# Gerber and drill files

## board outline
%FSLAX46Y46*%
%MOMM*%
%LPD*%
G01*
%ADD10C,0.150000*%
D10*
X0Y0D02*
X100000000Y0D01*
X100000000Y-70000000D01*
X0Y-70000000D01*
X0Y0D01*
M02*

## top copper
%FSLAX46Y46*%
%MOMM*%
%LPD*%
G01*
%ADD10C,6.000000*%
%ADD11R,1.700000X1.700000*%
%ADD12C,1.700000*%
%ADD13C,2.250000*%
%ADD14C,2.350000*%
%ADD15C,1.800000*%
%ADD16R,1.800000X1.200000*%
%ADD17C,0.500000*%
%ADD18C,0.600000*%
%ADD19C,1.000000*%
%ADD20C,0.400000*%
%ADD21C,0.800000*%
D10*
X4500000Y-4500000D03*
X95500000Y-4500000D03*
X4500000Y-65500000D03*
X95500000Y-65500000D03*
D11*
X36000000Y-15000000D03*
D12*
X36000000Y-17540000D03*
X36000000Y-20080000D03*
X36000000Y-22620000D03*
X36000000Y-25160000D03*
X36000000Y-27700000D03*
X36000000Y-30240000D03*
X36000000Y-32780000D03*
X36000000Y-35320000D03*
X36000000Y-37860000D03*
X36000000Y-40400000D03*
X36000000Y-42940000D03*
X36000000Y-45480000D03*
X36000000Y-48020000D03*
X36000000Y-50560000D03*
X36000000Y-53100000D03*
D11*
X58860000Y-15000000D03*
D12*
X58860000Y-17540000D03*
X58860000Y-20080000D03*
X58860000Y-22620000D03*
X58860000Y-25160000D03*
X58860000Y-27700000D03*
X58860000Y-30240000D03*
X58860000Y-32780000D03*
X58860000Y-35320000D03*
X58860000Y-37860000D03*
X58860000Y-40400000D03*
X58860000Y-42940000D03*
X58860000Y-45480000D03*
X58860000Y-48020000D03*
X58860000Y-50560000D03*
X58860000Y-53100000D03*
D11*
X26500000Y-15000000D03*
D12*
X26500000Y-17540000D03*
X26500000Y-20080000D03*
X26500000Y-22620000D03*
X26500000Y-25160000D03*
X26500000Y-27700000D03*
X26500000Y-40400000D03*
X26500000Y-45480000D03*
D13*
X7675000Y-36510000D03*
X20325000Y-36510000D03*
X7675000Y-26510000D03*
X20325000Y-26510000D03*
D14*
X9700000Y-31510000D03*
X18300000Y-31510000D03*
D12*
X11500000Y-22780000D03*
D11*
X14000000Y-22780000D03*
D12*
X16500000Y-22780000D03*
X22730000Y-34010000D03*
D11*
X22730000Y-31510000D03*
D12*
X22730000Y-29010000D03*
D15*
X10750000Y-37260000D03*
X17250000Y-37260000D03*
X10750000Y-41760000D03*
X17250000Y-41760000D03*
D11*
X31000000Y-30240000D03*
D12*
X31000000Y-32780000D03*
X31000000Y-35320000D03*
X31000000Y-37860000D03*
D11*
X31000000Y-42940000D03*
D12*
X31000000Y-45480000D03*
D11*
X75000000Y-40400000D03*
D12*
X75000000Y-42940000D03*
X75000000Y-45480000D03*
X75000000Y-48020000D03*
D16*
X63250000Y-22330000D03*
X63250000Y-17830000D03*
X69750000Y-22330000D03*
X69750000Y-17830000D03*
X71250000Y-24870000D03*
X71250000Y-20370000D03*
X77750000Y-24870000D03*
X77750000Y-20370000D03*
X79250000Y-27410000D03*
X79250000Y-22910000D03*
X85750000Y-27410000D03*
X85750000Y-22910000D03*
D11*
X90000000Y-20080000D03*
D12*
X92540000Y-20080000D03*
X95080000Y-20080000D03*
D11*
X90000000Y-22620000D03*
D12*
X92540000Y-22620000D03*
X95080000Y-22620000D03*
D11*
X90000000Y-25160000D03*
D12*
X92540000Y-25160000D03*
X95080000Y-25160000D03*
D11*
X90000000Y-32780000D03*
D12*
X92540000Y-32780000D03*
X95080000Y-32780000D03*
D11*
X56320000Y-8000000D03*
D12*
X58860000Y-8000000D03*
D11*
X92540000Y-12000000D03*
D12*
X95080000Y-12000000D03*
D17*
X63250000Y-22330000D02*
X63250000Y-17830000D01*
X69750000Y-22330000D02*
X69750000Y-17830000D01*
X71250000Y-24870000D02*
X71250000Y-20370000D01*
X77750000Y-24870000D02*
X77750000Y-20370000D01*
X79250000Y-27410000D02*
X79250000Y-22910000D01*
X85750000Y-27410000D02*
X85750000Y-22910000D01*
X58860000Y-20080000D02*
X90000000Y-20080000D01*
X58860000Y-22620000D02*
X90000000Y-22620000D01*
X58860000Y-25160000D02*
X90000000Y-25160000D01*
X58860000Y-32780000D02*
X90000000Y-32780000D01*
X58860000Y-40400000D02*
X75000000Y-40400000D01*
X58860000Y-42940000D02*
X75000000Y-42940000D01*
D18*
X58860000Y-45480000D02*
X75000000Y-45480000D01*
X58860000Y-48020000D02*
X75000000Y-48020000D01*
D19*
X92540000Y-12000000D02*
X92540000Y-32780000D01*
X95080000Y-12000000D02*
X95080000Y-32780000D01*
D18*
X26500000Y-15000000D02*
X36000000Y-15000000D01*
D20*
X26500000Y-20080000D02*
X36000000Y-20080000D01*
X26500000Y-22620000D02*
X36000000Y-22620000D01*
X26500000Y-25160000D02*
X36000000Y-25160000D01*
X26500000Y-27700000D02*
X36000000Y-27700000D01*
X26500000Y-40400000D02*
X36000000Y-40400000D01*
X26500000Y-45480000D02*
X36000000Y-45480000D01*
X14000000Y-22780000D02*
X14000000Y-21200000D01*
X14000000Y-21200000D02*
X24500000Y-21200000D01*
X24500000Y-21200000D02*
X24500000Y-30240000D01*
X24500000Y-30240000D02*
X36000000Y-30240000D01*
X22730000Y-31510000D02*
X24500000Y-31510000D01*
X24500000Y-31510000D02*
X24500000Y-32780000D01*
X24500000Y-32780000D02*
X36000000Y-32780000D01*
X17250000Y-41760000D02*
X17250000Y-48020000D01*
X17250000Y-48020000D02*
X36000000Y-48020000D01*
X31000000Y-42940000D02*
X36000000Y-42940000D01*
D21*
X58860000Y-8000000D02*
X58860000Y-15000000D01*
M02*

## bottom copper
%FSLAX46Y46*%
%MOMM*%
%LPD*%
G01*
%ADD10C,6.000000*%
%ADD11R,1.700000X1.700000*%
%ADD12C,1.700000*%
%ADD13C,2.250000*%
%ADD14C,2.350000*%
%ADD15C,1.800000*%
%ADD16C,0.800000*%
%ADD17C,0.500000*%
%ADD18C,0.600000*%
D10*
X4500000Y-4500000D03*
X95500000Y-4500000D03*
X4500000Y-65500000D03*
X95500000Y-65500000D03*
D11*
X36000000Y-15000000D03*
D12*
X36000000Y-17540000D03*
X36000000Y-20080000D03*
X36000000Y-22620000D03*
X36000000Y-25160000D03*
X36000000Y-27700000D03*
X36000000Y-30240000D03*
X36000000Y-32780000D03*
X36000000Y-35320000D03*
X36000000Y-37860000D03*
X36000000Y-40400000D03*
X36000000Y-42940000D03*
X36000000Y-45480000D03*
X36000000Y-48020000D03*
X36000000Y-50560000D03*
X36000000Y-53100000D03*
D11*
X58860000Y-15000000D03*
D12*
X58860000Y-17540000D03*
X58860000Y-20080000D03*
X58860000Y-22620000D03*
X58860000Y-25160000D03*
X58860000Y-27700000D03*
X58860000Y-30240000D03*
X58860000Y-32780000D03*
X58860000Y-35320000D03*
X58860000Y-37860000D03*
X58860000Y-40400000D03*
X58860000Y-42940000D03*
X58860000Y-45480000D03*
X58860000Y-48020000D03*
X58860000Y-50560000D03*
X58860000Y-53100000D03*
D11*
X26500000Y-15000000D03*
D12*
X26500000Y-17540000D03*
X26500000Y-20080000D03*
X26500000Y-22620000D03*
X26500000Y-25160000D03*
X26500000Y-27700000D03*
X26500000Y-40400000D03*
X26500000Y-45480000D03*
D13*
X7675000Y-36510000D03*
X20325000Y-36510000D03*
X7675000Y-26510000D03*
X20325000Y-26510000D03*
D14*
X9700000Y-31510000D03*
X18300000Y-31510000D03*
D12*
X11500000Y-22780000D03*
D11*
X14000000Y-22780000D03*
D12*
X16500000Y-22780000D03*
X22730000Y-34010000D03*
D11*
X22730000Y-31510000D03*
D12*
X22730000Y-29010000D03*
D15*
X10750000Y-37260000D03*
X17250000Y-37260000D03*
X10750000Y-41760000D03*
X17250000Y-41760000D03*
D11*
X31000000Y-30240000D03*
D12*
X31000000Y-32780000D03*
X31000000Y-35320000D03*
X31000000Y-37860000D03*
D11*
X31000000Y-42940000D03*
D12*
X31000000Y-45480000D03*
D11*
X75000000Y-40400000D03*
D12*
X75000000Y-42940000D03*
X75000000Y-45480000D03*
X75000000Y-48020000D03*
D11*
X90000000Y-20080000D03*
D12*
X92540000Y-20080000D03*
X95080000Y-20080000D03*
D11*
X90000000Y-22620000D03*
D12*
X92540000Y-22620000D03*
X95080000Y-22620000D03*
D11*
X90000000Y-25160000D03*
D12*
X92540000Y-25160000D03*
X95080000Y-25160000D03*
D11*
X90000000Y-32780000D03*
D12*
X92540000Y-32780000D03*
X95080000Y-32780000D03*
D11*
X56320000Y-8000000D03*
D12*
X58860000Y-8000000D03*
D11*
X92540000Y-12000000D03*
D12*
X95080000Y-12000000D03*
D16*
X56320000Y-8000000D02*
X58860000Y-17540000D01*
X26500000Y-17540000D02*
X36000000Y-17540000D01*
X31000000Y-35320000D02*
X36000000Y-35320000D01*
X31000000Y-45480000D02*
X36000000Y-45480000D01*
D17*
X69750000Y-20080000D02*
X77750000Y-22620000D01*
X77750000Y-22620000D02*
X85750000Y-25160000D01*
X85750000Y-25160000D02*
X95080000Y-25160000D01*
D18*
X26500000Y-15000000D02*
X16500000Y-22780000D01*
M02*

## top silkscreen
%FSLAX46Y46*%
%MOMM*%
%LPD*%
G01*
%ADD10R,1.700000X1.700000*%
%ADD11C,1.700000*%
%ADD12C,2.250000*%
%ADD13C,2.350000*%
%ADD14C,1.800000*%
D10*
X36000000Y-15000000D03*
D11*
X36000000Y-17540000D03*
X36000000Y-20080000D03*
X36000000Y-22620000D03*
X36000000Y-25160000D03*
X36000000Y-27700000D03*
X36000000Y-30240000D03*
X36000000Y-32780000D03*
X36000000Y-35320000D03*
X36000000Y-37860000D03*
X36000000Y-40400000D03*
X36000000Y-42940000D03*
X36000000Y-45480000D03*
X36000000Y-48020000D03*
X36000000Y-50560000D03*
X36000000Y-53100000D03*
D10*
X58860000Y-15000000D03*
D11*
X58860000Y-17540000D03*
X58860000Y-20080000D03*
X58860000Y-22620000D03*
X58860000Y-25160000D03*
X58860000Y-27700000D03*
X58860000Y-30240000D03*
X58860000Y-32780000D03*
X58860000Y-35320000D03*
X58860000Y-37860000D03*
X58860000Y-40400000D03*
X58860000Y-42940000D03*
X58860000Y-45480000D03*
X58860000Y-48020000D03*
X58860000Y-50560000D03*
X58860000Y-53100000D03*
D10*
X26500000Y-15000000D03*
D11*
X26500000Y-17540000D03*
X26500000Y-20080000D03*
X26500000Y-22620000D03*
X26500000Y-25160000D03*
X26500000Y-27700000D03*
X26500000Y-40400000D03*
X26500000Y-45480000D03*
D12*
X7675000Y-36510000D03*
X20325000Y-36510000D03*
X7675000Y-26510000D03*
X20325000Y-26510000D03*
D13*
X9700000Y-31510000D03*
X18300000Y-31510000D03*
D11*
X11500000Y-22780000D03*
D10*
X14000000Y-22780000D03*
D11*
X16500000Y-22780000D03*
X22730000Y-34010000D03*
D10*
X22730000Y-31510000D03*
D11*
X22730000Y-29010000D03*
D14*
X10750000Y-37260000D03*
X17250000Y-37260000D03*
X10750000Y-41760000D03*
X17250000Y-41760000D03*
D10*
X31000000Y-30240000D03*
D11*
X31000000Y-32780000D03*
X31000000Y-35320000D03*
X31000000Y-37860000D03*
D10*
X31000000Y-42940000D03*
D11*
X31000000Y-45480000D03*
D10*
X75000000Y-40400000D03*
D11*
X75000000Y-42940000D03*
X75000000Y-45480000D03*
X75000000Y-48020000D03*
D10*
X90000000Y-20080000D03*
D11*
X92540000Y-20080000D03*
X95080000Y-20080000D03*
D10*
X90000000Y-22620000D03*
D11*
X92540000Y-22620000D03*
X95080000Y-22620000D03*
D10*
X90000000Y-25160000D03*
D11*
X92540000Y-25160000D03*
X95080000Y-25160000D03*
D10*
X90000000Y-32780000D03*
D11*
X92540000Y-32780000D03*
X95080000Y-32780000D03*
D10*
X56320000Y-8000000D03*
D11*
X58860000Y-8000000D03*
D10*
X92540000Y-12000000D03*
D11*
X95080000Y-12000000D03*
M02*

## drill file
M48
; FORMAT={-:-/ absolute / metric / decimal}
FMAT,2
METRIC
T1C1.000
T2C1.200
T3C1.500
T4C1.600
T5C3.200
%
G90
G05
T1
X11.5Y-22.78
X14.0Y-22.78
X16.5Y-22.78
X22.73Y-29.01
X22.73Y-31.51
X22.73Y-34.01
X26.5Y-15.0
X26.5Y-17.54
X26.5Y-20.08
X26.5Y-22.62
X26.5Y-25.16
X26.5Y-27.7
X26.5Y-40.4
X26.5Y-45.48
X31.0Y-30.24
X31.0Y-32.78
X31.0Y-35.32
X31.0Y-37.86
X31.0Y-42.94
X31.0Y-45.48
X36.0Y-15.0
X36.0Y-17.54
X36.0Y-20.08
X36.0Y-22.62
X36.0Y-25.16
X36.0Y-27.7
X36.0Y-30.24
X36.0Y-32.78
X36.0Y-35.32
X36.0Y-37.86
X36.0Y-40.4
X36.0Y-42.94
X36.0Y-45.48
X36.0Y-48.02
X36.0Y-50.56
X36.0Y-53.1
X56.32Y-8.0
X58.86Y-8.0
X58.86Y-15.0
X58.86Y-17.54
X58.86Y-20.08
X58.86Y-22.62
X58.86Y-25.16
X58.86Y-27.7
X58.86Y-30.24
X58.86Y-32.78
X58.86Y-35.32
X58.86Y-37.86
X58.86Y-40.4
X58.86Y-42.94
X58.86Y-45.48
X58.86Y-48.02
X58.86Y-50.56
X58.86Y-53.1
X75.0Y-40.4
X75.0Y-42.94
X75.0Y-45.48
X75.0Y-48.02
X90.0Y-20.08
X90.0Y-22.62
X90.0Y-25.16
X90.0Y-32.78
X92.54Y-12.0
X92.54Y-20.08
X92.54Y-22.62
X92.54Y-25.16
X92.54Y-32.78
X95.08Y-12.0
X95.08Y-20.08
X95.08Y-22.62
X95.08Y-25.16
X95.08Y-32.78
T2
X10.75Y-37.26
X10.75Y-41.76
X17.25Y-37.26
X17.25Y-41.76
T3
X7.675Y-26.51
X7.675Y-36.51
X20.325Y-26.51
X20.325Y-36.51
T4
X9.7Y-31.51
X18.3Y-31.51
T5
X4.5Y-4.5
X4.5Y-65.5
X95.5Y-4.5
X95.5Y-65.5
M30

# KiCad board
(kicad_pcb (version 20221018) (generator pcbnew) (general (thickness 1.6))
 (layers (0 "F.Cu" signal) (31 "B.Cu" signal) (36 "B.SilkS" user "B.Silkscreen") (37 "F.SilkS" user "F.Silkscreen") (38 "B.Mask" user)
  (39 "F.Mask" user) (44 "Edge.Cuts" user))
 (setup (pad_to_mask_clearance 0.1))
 (gr_rect (start 0 0) (end 100.0 70.0) (layer "Edge.Cuts") (width 0.15) (fill none))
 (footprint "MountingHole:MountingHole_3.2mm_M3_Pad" (layer "F.Cu") (at 4.5 4.5)
  (pad "" np_thru_hole circle (at 0 0) (size 6.0 6.0) (drill 3.2) (layers *.Cu *.Mask)))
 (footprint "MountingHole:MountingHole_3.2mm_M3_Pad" (layer "F.Cu") (at 95.5 4.5)
  (pad "" np_thru_hole circle (at 0 0) (size 6.0 6.0) (drill 3.2) (layers *.Cu *.Mask)))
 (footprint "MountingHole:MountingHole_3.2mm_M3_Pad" (layer "F.Cu") (at 4.5 65.5)
  (pad "" np_thru_hole circle (at 0 0) (size 6.0 6.0) (drill 3.2) (layers *.Cu *.Mask)))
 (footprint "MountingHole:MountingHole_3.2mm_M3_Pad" (layer "F.Cu") (at 95.5 65.5)
  (pad "" np_thru_hole circle (at 0 0) (size 6.0 6.0) (drill 3.2) (layers *.Cu *.Mask)))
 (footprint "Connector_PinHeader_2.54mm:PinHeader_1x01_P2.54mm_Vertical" (layer "F.Cu") (at 36.0 15.0)
  (pad "1" thru_hole rect (at 0 0) (size 1.7 1.7) (drill 1.0) (layers *.Cu *.Mask "F.SilkS")))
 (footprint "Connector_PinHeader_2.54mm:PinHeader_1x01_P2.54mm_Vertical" (layer "F.Cu") (at 36.0 17.54)
  (pad "1" thru_hole circle (at 0 0) (size 1.7 1.7) (drill 1.0) (layers *.Cu *.Mask "F.SilkS")))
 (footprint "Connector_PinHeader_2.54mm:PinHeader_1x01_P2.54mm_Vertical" (layer "F.Cu") (at 36.0 20.08)
  (pad "1" thru_hole circle (at 0 0) (size 1.7 1.7) (drill 1.0) (layers *.Cu *.Mask "F.SilkS")))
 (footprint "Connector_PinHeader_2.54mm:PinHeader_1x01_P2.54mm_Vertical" (layer "F.Cu") (at 36.0 22.62)
  (pad "1" thru_hole circle (at 0 0) (size 1.7 1.7) (drill 1.0) (layers *.Cu *.Mask "F.SilkS")))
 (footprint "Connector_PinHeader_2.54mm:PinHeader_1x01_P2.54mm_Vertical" (layer "F.Cu") (at 36.0 25.16)
  (pad "1" thru_hole circle (at 0 0) (size 1.7 1.7) (drill 1.0) (layers *.Cu *.Mask "F.SilkS")))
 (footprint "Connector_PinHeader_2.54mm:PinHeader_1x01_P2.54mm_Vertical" (layer "F.Cu") (at 36.0 27.7)
  (pad "1" thru_hole circle (at 0 0) (size 1.7 1.7) (drill 1.0) (layers *.Cu *.Mask "F.SilkS")))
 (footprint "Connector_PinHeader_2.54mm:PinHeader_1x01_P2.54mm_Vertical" (layer "F.Cu") (at 36.0 30.240000000000002)
  (pad "1" thru_hole circle (at 0 0) (size 1.7 1.7) (drill 1.0) (layers *.Cu *.Mask "F.SilkS")))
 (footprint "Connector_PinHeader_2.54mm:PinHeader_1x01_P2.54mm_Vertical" (layer "F.Cu") (at 36.0 32.78)
  (pad "1" thru_hole circle (at 0 0) (size 1.7 1.7) (drill 1.0) (layers *.Cu *.Mask "F.SilkS")))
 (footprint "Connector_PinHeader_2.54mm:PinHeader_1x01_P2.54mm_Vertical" (layer "F.Cu") (at 36.0 35.32)
  (pad "1" thru_hole circle (at 0 0) (size 1.7 1.7) (drill 1.0) (layers *.Cu *.Mask "F.SilkS")))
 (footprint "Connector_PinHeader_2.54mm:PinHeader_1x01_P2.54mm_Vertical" (layer "F.Cu") (at 36.0 37.86)
  (pad "1" thru_hole circle (at 0 0) (size 1.7 1.7) (drill 1.0) (layers *.Cu *.Mask "F.SilkS")))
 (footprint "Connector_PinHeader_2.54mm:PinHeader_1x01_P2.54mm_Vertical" (layer "F.Cu") (at 36.0 40.4)
  (pad "1" thru_hole circle (at 0 0) (size 1.7 1.7) (drill 1.0) (layers *.Cu *.Mask "F.SilkS")))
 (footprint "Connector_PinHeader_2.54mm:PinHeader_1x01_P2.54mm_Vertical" (layer "F.Cu") (at 36.0 42.94)
  (pad "1" thru_hole circle (at 0 0) (size 1.7 1.7) (drill 1.0) (layers *.Cu *.Mask "F.SilkS")))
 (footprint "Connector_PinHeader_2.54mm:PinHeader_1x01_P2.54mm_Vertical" (layer "F.Cu") (at 36.0 45.480000000000004)
  (pad "1" thru_hole circle (at 0 0) (size 1.7 1.7) (drill 1.0) (layers *.Cu *.Mask "F.SilkS")))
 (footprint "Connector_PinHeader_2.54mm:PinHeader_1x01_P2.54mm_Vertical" (layer "F.Cu") (at 36.0 48.02)
  (pad "1" thru_hole circle (at 0 0) (size 1.7 1.7) (drill 1.0) (layers *.Cu *.Mask "F.SilkS")))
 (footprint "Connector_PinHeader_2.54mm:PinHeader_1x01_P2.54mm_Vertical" (layer "F.Cu") (at 36.0 50.56)
  (pad "1" thru_hole circle (at 0 0) (size 1.7 1.7) (drill 1.0) (layers *.Cu *.Mask "F.SilkS")))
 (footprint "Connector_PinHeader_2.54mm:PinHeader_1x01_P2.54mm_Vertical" (layer "F.Cu") (at 36.0 53.1)
  (pad "1" thru_hole circle (at 0 0) (size 1.7 1.7) (drill 1.0) (layers *.Cu *.Mask "F.SilkS")))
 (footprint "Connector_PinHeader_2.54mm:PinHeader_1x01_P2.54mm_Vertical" (layer "F.Cu") (at 58.86 15.0)
  (pad "1" thru_hole rect (at 0 0) (size 1.7 1.7) (drill 1.0) (layers *.Cu *.Mask "F.SilkS")))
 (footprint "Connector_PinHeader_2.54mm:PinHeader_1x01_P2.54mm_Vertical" (layer "F.Cu") (at 58.86 17.54)
  (pad "1" thru_hole circle (at 0 0) (size 1.7 1.7) (drill 1.0) (layers *.Cu *.Mask "F.SilkS")))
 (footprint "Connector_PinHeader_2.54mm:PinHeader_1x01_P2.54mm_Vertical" (layer "F.Cu") (at 58.86 20.08)
  (pad "1" thru_hole circle (at 0 0) (size 1.7 1.7) (drill 1.0) (layers *.Cu *.Mask "F.SilkS")))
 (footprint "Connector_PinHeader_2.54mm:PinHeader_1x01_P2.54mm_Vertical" (layer "F.Cu") (at 58.86 22.62)
  (pad "1" thru_hole circle (at 0 0) (size 1.7 1.7) (drill 1.0) (layers *.Cu *.Mask "F.SilkS")))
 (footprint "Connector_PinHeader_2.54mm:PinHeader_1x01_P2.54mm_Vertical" (layer "F.Cu") (at 58.86 25.16)
  (pad "1" thru_hole circle (at 0 0) (size 1.7 1.7) (drill 1.0) (layers *.Cu *.Mask "F.SilkS")))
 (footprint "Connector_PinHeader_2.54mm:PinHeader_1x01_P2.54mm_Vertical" (layer "F.Cu") (at 58.86 27.7)
  (pad "1" thru_hole circle (at 0 0) (size 1.7 1.7) (drill 1.0) (layers *.Cu *.Mask "F.SilkS")))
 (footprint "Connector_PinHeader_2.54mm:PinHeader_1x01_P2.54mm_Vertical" (layer "F.Cu") (at 58.86 30.240000000000002)
  (pad "1" thru_hole circle (at 0 0) (size 1.7 1.7) (drill 1.0) (layers *.Cu *.Mask "F.SilkS")))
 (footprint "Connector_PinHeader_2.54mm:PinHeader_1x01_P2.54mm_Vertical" (layer "F.Cu") (at 58.86 32.78)
  (pad "1" thru_hole circle (at 0 0) (size 1.7 1.7) (drill 1.0) (layers *.Cu *.Mask "F.SilkS")))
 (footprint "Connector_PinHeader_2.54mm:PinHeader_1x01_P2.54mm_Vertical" (layer "F.Cu") (at 58.86 35.32)
  (pad "1" thru_hole circle (at 0 0) (size 1.7 1.7) (drill 1.0) (layers *.Cu *.Mask "F.SilkS")))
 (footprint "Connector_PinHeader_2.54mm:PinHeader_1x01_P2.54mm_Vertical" (layer "F.Cu") (at 58.86 37.86)
  (pad "1" thru_hole circle (at 0 0) (size 1.7 1.7) (drill 1.0) (layers *.Cu *.Mask "F.SilkS")))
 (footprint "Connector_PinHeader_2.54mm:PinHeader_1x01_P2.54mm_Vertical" (layer "F.Cu") (at 58.86 40.4)
  (pad "1" thru_hole circle (at 0 0) (size 1.7 1.7) (drill 1.0) (layers *.Cu *.Mask "F.SilkS")))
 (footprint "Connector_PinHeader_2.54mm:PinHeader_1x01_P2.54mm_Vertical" (layer "F.Cu") (at 58.86 42.94)
  (pad "1" thru_hole circle (at 0 0) (size 1.7 1.7) (drill 1.0) (layers *.Cu *.Mask "F.SilkS")))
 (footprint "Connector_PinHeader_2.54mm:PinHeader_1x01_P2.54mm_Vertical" (layer "F.Cu") (at 58.86 45.480000000000004)
  (pad "1" thru_hole circle (at 0 0) (size 1.7 1.7) (drill 1.0) (layers *.Cu *.Mask "F.SilkS")))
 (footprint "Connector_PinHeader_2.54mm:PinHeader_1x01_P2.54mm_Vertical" (layer "F.Cu") (at 58.86 48.02)
  (pad "1" thru_hole circle (at 0 0) (size 1.7 1.7) (drill 1.0) (layers *.Cu *.Mask "F.SilkS")))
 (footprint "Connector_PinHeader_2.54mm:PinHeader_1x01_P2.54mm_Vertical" (layer "F.Cu") (at 58.86 50.56)
  (pad "1" thru_hole circle (at 0 0) (size 1.7 1.7) (drill 1.0) (layers *.Cu *.Mask "F.SilkS")))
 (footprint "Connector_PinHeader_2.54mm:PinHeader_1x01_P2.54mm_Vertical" (layer "F.Cu") (at 58.86 53.1)
  (pad "1" thru_hole circle (at 0 0) (size 1.7 1.7) (drill 1.0) (layers *.Cu *.Mask "F.SilkS")))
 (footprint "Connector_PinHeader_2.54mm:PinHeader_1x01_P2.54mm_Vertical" (layer "F.Cu") (at 26.5 15.0)
  (pad "1" thru_hole rect (at 0 0) (size 1.7 1.7) (drill 1.0) (layers *.Cu *.Mask "F.SilkS")))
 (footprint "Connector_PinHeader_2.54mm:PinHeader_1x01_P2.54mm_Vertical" (layer "F.Cu") (at 26.5 17.54)
  (pad "1" thru_hole circle (at 0 0) (size 1.7 1.7) (drill 1.0) (layers *.Cu *.Mask "F.SilkS")))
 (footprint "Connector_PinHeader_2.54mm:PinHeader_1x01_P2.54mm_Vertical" (layer "F.Cu") (at 26.5 20.08)
  (pad "1" thru_hole circle (at 0 0) (size 1.7 1.7) (drill 1.0) (layers *.Cu *.Mask "F.SilkS")))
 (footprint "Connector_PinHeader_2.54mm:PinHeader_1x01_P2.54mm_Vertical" (layer "F.Cu") (at 26.5 22.62)
  (pad "1" thru_hole circle (at 0 0) (size 1.7 1.7) (drill 1.0) (layers *.Cu *.Mask "F.SilkS")))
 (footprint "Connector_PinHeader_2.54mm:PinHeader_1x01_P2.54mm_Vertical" (layer "F.Cu") (at 26.5 25.16)
  (pad "1" thru_hole circle (at 0 0) (size 1.7 1.7) (drill 1.0) (layers *.Cu *.Mask "F.SilkS")))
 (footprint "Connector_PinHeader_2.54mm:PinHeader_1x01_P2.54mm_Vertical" (layer "F.Cu") (at 26.5 27.7)
  (pad "1" thru_hole circle (at 0 0) (size 1.7 1.7) (drill 1.0) (layers *.Cu *.Mask "F.SilkS")))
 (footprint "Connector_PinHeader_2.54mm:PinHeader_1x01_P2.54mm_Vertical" (layer "F.Cu") (at 26.5 40.4)
  (pad "1" thru_hole circle (at 0 0) (size 1.7 1.7) (drill 1.0) (layers *.Cu *.Mask "F.SilkS")))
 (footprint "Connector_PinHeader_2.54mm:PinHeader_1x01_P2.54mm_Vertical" (layer "F.Cu") (at 26.5 45.48)
  (pad "1" thru_hole circle (at 0 0) (size 1.7 1.7) (drill 1.0) (layers *.Cu *.Mask "F.SilkS")))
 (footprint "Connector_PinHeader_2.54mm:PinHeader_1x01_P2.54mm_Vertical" (layer "F.Cu") (at 7.675 36.510000000000005)
  (pad "1" thru_hole circle (at 0 0) (size 2.25 2.25) (drill 1.5) (layers *.Cu *.Mask "F.SilkS")))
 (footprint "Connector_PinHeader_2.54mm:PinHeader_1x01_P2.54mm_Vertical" (layer "F.Cu") (at 20.325 36.510000000000005)
  (pad "1" thru_hole circle (at 0 0) (size 2.25 2.25) (drill 1.5) (layers *.Cu *.Mask "F.SilkS")))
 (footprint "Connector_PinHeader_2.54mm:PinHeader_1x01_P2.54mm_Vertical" (layer "F.Cu") (at 7.675 26.51)
  (pad "1" thru_hole circle (at 0 0) (size 2.25 2.25) (drill 1.5) (layers *.Cu *.Mask "F.SilkS")))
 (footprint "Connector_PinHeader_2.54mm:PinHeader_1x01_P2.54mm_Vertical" (layer "F.Cu") (at 20.325 26.51)
  (pad "1" thru_hole circle (at 0 0) (size 2.25 2.25) (drill 1.5) (layers *.Cu *.Mask "F.SilkS")))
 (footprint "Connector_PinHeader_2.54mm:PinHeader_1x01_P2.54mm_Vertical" (layer "F.Cu") (at 9.7 31.51)
  (pad "1" thru_hole circle (at 0 0) (size 2.35 2.35) (drill 1.6) (layers *.Cu *.Mask "F.SilkS")))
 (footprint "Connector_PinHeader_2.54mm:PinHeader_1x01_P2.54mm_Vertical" (layer "F.Cu") (at 18.3 31.51)
  (pad "1" thru_hole circle (at 0 0) (size 2.35 2.35) (drill 1.6) (layers *.Cu *.Mask "F.SilkS")))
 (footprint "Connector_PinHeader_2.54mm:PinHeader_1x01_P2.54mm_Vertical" (layer "F.Cu") (at 11.5 22.78)
  (pad "1" thru_hole circle (at 0 0) (size 1.7 1.7) (drill 1.0) (layers *.Cu *.Mask "F.SilkS")))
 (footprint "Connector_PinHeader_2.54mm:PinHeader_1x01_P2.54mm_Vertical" (layer "F.Cu") (at 14.0 22.78)
  (pad "1" thru_hole rect (at 0 0) (size 1.7 1.7) (drill 1.0) (layers *.Cu *.Mask "F.SilkS")))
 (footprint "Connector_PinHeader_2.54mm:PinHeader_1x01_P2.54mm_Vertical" (layer "F.Cu") (at 16.5 22.78)
  (pad "1" thru_hole circle (at 0 0) (size 1.7 1.7) (drill 1.0) (layers *.Cu *.Mask "F.SilkS")))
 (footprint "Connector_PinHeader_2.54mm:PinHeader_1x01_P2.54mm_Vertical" (layer "F.Cu") (at 22.73 34.010000000000005)
  (pad "1" thru_hole circle (at 0 0) (size 1.7 1.7) (drill 1.0) (layers *.Cu *.Mask "F.SilkS")))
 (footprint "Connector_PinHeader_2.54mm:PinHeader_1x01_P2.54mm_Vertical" (layer "F.Cu") (at 22.73 31.51)
  (pad "1" thru_hole rect (at 0 0) (size 1.7 1.7) (drill 1.0) (layers *.Cu *.Mask "F.SilkS")))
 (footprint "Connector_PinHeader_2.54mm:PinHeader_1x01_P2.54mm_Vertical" (layer "F.Cu") (at 22.73 29.01)
  (pad "1" thru_hole circle (at 0 0) (size 1.7 1.7) (drill 1.0) (layers *.Cu *.Mask "F.SilkS")))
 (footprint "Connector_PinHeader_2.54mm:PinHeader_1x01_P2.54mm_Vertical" (layer "F.Cu") (at 10.75 37.260000000000005)
  (pad "1" thru_hole circle (at 0 0) (size 1.8 1.8) (drill 1.2) (layers *.Cu *.Mask "F.SilkS")))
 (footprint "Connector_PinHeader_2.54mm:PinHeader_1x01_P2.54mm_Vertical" (layer "F.Cu") (at 17.25 37.260000000000005)
  (pad "1" thru_hole circle (at 0 0) (size 1.8 1.8) (drill 1.2) (layers *.Cu *.Mask "F.SilkS")))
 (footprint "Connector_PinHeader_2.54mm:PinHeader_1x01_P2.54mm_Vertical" (layer "F.Cu") (at 10.75 41.760000000000005)
  (pad "1" thru_hole circle (at 0 0) (size 1.8 1.8) (drill 1.2) (layers *.Cu *.Mask "F.SilkS")))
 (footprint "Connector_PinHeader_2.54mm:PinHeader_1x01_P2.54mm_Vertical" (layer "F.Cu") (at 17.25 41.760000000000005)
  (pad "1" thru_hole circle (at 0 0) (size 1.8 1.8) (drill 1.2) (layers *.Cu *.Mask "F.SilkS")))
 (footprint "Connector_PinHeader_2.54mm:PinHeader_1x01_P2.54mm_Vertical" (layer "F.Cu") (at 31.0 30.24)
  (pad "1" thru_hole rect (at 0 0) (size 1.7 1.7) (drill 1.0) (layers *.Cu *.Mask "F.SilkS")))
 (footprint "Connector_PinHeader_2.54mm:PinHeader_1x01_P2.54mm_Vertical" (layer "F.Cu") (at 31.0 32.78)
  (pad "1" thru_hole circle (at 0 0) (size 1.7 1.7) (drill 1.0) (layers *.Cu *.Mask "F.SilkS")))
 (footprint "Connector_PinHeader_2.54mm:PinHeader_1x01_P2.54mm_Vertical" (layer "F.Cu") (at 31.0 35.32)
  (pad "1" thru_hole circle (at 0 0) (size 1.7 1.7) (drill 1.0) (layers *.Cu *.Mask "F.SilkS")))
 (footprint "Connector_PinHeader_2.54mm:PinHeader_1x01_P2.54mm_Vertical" (layer "F.Cu") (at 31.0 37.86)
  (pad "1" thru_hole circle (at 0 0) (size 1.7 1.7) (drill 1.0) (layers *.Cu *.Mask "F.SilkS")))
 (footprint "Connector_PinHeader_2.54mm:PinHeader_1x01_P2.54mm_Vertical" (layer "F.Cu") (at 31.0 42.94)
  (pad "1" thru_hole rect (at 0 0) (size 1.7 1.7) (drill 1.0) (layers *.Cu *.Mask "F.SilkS")))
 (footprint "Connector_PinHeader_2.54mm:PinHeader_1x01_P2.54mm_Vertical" (layer "F.Cu") (at 31.0 45.48)
  (pad "1" thru_hole circle (at 0 0) (size 1.7 1.7) (drill 1.0) (layers *.Cu *.Mask "F.SilkS")))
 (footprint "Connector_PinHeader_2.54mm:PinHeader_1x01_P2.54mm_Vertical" (layer "F.Cu") (at 75.0 40.4)
  (pad "1" thru_hole rect (at 0 0) (size 1.7 1.7) (drill 1.0) (layers *.Cu *.Mask "F.SilkS")))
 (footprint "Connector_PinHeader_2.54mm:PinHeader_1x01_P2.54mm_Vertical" (layer "F.Cu") (at 75.0 42.94)
  (pad "1" thru_hole circle (at 0 0) (size 1.7 1.7) (drill 1.0) (layers *.Cu *.Mask "F.SilkS")))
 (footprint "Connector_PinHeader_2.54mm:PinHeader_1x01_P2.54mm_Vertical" (layer "F.Cu") (at 75.0 45.48)
  (pad "1" thru_hole circle (at 0 0) (size 1.7 1.7) (drill 1.0) (layers *.Cu *.Mask "F.SilkS")))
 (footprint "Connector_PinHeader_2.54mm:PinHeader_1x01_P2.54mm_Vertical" (layer "F.Cu") (at 75.0 48.019999999999996)
  (pad "1" thru_hole circle (at 0 0) (size 1.7 1.7) (drill 1.0) (layers *.Cu *.Mask "F.SilkS")))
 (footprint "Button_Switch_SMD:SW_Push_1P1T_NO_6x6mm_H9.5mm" (layer "F.Cu") (at 63.25 22.33)
  (pad "1" smd rect (at 0 0) (size 1.8 1.2) (layers "F.Cu" "F.Mask")))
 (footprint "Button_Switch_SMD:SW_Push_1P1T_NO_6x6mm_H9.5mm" (layer "F.Cu") (at 63.25 17.83)
  (pad "1" smd rect (at 0 0) (size 1.8 1.2) (layers "F.Cu" "F.Mask")))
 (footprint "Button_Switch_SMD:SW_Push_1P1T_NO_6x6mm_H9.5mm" (layer "F.Cu") (at 69.75 22.33)
  (pad "1" smd rect (at 0 0) (size 1.8 1.2) (layers "F.Cu" "F.Mask")))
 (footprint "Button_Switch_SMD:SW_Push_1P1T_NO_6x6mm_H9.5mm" (layer "F.Cu") (at 69.75 17.83)
  (pad "1" smd rect (at 0 0) (size 1.8 1.2) (layers "F.Cu" "F.Mask")))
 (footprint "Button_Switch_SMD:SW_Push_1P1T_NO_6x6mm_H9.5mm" (layer "F.Cu") (at 71.25 24.87)
  (pad "1" smd rect (at 0 0) (size 1.8 1.2) (layers "F.Cu" "F.Mask")))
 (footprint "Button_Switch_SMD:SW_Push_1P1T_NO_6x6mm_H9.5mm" (layer "F.Cu") (at 71.25 20.37)
  (pad "1" smd rect (at 0 0) (size 1.8 1.2) (layers "F.Cu" "F.Mask")))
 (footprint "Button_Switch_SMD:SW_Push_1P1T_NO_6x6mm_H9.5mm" (layer "F.Cu") (at 77.75 24.87)
  (pad "1" smd rect (at 0 0) (size 1.8 1.2) (layers "F.Cu" "F.Mask")))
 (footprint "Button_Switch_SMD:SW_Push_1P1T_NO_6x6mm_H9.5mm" (layer "F.Cu") (at 77.75 20.37)
  (pad "1" smd rect (at 0 0) (size 1.8 1.2) (layers "F.Cu" "F.Mask")))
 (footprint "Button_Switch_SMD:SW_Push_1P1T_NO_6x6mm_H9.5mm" (layer "F.Cu") (at 79.25 27.41)
  (pad "1" smd rect (at 0 0) (size 1.8 1.2) (layers "F.Cu" "F.Mask")))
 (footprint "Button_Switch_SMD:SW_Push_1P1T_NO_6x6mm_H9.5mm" (layer "F.Cu") (at 79.25 22.91)
  (pad "1" smd rect (at 0 0) (size 1.8 1.2) (layers "F.Cu" "F.Mask")))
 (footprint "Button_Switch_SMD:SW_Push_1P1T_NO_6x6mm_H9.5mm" (layer "F.Cu") (at 85.75 27.41)
  (pad "1" smd rect (at 0 0) (size 1.8 1.2) (layers "F.Cu" "F.Mask")))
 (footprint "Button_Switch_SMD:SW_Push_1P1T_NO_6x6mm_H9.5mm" (layer "F.Cu") (at 85.75 22.91)
  (pad "1" smd rect (at 0 0) (size 1.8 1.2) (layers "F.Cu" "F.Mask")))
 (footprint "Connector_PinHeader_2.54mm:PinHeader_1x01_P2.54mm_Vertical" (layer "F.Cu") (at 90.0 20.08)
  (pad "1" thru_hole rect (at 0 0) (size 1.7 1.7) (drill 1.0) (layers *.Cu *.Mask "F.SilkS")))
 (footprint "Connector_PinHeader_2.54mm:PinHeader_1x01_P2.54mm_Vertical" (layer "F.Cu") (at 92.54 20.08)
  (pad "1" thru_hole circle (at 0 0) (size 1.7 1.7) (drill 1.0) (layers *.Cu *.Mask "F.SilkS")))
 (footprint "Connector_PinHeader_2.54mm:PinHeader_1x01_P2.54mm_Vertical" (layer "F.Cu") (at 95.08 20.08)
  (pad "1" thru_hole circle (at 0 0) (size 1.7 1.7) (drill 1.0) (layers *.Cu *.Mask "F.SilkS")))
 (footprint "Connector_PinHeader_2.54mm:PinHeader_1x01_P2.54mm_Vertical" (layer "F.Cu") (at 90.0 22.62)
  (pad "1" thru_hole rect (at 0 0) (size 1.7 1.7) (drill 1.0) (layers *.Cu *.Mask "F.SilkS")))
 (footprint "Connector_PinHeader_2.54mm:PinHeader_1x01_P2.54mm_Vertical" (layer "F.Cu") (at 92.54 22.62)
  (pad "1" thru_hole circle (at 0 0) (size 1.7 1.7) (drill 1.0) (layers *.Cu *.Mask "F.SilkS")))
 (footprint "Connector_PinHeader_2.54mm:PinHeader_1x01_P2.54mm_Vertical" (layer "F.Cu") (at 95.08 22.62)
  (pad "1" thru_hole circle (at 0 0) (size 1.7 1.7) (drill 1.0) (layers *.Cu *.Mask "F.SilkS")))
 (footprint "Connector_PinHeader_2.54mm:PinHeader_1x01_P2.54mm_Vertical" (layer "F.Cu") (at 90.0 25.16)
  (pad "1" thru_hole rect (at 0 0) (size 1.7 1.7) (drill 1.0) (layers *.Cu *.Mask "F.SilkS")))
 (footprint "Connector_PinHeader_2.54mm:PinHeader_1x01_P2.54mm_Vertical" (layer "F.Cu") (at 92.54 25.16)
  (pad "1" thru_hole circle (at 0 0) (size 1.7 1.7) (drill 1.0) (layers *.Cu *.Mask "F.SilkS")))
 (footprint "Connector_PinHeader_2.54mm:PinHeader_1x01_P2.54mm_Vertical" (layer "F.Cu") (at 95.08 25.16)
  (pad "1" thru_hole circle (at 0 0) (size 1.7 1.7) (drill 1.0) (layers *.Cu *.Mask "F.SilkS")))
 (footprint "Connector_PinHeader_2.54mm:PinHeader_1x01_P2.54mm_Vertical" (layer "F.Cu") (at 90.0 32.78)
  (pad "1" thru_hole rect (at 0 0) (size 1.7 1.7) (drill 1.0) (layers *.Cu *.Mask "F.SilkS")))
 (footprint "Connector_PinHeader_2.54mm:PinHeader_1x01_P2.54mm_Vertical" (layer "F.Cu") (at 92.54 32.78)
  (pad "1" thru_hole circle (at 0 0) (size 1.7 1.7) (drill 1.0) (layers *.Cu *.Mask "F.SilkS")))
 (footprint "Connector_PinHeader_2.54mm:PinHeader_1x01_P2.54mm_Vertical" (layer "F.Cu") (at 95.08 32.78)
  (pad "1" thru_hole circle (at 0 0) (size 1.7 1.7) (drill 1.0) (layers *.Cu *.Mask "F.SilkS")))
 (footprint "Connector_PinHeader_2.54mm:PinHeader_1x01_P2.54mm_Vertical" (layer "F.Cu") (at 56.32 8.0)
  (pad "1" thru_hole rect (at 0 0) (size 1.7 1.7) (drill 1.0) (layers *.Cu *.Mask "F.SilkS")))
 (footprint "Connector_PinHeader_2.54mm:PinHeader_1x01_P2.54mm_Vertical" (layer "F.Cu") (at 58.86 8.0)
  (pad "1" thru_hole circle (at 0 0) (size 1.7 1.7) (drill 1.0) (layers *.Cu *.Mask "F.SilkS")))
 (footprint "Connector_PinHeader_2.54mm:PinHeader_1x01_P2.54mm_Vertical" (layer "F.Cu") (at 92.54 12.0)
  (pad "1" thru_hole rect (at 0 0) (size 1.7 1.7) (drill 1.0) (layers *.Cu *.Mask "F.SilkS")))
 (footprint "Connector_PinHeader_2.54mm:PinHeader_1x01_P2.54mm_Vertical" (layer "F.Cu") (at 95.08000000000001 12.0)
  (pad "1" thru_hole circle (at 0 0) (size 1.7 1.7) (drill 1.0) (layers *.Cu *.Mask "F.SilkS")))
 (segment (start 63.25 22.33) (end 63.25 17.83) (width 0.5) (layer "F.Cu") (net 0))
 (segment (start 69.75 22.33) (end 69.75 17.83) (width 0.5) (layer "F.Cu") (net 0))
 (segment (start 71.25 24.87) (end 71.25 20.37) (width 0.5) (layer "F.Cu") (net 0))
 (segment (start 77.75 24.87) (end 77.75 20.37) (width 0.5) (layer "F.Cu") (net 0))
 (segment (start 79.25 27.41) (end 79.25 22.91) (width 0.5) (layer "F.Cu") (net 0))
 (segment (start 85.75 27.41) (end 85.75 22.91) (width 0.5) (layer "F.Cu") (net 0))
 (segment (start 58.86 20.08) (end 90.0 20.08) (width 0.5) (layer "F.Cu") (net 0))
 (segment (start 58.86 22.62) (end 90.0 22.62) (width 0.5) (layer "F.Cu") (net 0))
 (segment (start 58.86 25.16) (end 90.0 25.16) (width 0.5) (layer "F.Cu") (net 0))
 (segment (start 58.86 32.78) (end 90.0 32.78) (width 0.5) (layer "F.Cu") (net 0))
 (segment (start 58.86 40.4) (end 75.0 40.4) (width 0.5) (layer "F.Cu") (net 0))
 (segment (start 58.86 42.94) (end 75.0 42.94) (width 0.5) (layer "F.Cu") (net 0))
 (segment (start 58.86 45.48) (end 75.0 45.48) (width 0.6) (layer "F.Cu") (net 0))
 (segment (start 58.86 48.02) (end 75.0 48.02) (width 0.6) (layer "F.Cu") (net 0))
 (segment (start 92.54 12.0) (end 92.54 32.78) (width 1.0) (layer "F.Cu") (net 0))
 (segment (start 95.08 12.0) (end 95.08 32.78) (width 1.0) (layer "F.Cu") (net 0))
 (segment (start 26.5 15.0) (end 36.0 15.0) (width 0.6) (layer "F.Cu") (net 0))
 (segment (start 26.5 20.08) (end 36.0 20.08) (width 0.4) (layer "F.Cu") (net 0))
 (segment (start 26.5 22.62) (end 36.0 22.62) (width 0.4) (layer "F.Cu") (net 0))
 (segment (start 26.5 25.16) (end 36.0 25.16) (width 0.4) (layer "F.Cu") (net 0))
 (segment (start 26.5 27.7) (end 36.0 27.7) (width 0.4) (layer "F.Cu") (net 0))
 (segment (start 26.5 40.4) (end 36.0 40.4) (width 0.4) (layer "F.Cu") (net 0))
 (segment (start 26.5 45.48) (end 36.0 45.48) (width 0.4) (layer "F.Cu") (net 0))
 (segment (start 14.0 22.78) (end 14.0 21.2) (width 0.4) (layer "F.Cu") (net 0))
 (segment (start 14.0 21.2) (end 24.5 21.2) (width 0.4) (layer "F.Cu") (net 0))
 (segment (start 24.5 21.2) (end 24.5 30.24) (width 0.4) (layer "F.Cu") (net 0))
 (segment (start 24.5 30.24) (end 36.0 30.24) (width 0.4) (layer "F.Cu") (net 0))
 (segment (start 22.73 31.51) (end 24.5 31.51) (width 0.4) (layer "F.Cu") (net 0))
 (segment (start 24.5 31.51) (end 24.5 32.78) (width 0.4) (layer "F.Cu") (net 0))
 (segment (start 24.5 32.78) (end 36.0 32.78) (width 0.4) (layer "F.Cu") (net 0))
 (segment (start 17.25 41.76) (end 17.25 48.02) (width 0.4) (layer "F.Cu") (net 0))
 (segment (start 17.25 48.02) (end 36.0 48.02) (width 0.4) (layer "F.Cu") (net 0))
 (segment (start 31.0 42.94) (end 36.0 42.94) (width 0.4) (layer "F.Cu") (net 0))
 (segment (start 58.86 8.0) (end 58.86 15.0) (width 0.8) (layer "F.Cu") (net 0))
 (segment (start 56.32 8.0) (end 58.86 17.54) (width 0.8) (layer "B.Cu") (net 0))
 (segment (start 26.5 17.54) (end 36.0 17.54) (width 0.8) (layer "B.Cu") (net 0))
 (segment (start 31.0 35.32) (end 36.0 35.32) (width 0.8) (layer "B.Cu") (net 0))
 (segment (start 31.0 45.48) (end 36.0 45.48) (width 0.8) (layer "B.Cu") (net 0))
 (segment (start 69.75 20.08) (end 77.75 22.62) (width 0.5) (layer "B.Cu") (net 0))
 (segment (start 77.75 22.62) (end 85.75 25.16) (width 0.5) (layer "B.Cu") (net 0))
 (segment (start 85.75 25.16) (end 95.08 25.16) (width 0.5) (layer "B.Cu") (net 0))
 (segment (start 26.5 15.0) (end 16.5 22.78) (width 0.6) (layer "B.Cu") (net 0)))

